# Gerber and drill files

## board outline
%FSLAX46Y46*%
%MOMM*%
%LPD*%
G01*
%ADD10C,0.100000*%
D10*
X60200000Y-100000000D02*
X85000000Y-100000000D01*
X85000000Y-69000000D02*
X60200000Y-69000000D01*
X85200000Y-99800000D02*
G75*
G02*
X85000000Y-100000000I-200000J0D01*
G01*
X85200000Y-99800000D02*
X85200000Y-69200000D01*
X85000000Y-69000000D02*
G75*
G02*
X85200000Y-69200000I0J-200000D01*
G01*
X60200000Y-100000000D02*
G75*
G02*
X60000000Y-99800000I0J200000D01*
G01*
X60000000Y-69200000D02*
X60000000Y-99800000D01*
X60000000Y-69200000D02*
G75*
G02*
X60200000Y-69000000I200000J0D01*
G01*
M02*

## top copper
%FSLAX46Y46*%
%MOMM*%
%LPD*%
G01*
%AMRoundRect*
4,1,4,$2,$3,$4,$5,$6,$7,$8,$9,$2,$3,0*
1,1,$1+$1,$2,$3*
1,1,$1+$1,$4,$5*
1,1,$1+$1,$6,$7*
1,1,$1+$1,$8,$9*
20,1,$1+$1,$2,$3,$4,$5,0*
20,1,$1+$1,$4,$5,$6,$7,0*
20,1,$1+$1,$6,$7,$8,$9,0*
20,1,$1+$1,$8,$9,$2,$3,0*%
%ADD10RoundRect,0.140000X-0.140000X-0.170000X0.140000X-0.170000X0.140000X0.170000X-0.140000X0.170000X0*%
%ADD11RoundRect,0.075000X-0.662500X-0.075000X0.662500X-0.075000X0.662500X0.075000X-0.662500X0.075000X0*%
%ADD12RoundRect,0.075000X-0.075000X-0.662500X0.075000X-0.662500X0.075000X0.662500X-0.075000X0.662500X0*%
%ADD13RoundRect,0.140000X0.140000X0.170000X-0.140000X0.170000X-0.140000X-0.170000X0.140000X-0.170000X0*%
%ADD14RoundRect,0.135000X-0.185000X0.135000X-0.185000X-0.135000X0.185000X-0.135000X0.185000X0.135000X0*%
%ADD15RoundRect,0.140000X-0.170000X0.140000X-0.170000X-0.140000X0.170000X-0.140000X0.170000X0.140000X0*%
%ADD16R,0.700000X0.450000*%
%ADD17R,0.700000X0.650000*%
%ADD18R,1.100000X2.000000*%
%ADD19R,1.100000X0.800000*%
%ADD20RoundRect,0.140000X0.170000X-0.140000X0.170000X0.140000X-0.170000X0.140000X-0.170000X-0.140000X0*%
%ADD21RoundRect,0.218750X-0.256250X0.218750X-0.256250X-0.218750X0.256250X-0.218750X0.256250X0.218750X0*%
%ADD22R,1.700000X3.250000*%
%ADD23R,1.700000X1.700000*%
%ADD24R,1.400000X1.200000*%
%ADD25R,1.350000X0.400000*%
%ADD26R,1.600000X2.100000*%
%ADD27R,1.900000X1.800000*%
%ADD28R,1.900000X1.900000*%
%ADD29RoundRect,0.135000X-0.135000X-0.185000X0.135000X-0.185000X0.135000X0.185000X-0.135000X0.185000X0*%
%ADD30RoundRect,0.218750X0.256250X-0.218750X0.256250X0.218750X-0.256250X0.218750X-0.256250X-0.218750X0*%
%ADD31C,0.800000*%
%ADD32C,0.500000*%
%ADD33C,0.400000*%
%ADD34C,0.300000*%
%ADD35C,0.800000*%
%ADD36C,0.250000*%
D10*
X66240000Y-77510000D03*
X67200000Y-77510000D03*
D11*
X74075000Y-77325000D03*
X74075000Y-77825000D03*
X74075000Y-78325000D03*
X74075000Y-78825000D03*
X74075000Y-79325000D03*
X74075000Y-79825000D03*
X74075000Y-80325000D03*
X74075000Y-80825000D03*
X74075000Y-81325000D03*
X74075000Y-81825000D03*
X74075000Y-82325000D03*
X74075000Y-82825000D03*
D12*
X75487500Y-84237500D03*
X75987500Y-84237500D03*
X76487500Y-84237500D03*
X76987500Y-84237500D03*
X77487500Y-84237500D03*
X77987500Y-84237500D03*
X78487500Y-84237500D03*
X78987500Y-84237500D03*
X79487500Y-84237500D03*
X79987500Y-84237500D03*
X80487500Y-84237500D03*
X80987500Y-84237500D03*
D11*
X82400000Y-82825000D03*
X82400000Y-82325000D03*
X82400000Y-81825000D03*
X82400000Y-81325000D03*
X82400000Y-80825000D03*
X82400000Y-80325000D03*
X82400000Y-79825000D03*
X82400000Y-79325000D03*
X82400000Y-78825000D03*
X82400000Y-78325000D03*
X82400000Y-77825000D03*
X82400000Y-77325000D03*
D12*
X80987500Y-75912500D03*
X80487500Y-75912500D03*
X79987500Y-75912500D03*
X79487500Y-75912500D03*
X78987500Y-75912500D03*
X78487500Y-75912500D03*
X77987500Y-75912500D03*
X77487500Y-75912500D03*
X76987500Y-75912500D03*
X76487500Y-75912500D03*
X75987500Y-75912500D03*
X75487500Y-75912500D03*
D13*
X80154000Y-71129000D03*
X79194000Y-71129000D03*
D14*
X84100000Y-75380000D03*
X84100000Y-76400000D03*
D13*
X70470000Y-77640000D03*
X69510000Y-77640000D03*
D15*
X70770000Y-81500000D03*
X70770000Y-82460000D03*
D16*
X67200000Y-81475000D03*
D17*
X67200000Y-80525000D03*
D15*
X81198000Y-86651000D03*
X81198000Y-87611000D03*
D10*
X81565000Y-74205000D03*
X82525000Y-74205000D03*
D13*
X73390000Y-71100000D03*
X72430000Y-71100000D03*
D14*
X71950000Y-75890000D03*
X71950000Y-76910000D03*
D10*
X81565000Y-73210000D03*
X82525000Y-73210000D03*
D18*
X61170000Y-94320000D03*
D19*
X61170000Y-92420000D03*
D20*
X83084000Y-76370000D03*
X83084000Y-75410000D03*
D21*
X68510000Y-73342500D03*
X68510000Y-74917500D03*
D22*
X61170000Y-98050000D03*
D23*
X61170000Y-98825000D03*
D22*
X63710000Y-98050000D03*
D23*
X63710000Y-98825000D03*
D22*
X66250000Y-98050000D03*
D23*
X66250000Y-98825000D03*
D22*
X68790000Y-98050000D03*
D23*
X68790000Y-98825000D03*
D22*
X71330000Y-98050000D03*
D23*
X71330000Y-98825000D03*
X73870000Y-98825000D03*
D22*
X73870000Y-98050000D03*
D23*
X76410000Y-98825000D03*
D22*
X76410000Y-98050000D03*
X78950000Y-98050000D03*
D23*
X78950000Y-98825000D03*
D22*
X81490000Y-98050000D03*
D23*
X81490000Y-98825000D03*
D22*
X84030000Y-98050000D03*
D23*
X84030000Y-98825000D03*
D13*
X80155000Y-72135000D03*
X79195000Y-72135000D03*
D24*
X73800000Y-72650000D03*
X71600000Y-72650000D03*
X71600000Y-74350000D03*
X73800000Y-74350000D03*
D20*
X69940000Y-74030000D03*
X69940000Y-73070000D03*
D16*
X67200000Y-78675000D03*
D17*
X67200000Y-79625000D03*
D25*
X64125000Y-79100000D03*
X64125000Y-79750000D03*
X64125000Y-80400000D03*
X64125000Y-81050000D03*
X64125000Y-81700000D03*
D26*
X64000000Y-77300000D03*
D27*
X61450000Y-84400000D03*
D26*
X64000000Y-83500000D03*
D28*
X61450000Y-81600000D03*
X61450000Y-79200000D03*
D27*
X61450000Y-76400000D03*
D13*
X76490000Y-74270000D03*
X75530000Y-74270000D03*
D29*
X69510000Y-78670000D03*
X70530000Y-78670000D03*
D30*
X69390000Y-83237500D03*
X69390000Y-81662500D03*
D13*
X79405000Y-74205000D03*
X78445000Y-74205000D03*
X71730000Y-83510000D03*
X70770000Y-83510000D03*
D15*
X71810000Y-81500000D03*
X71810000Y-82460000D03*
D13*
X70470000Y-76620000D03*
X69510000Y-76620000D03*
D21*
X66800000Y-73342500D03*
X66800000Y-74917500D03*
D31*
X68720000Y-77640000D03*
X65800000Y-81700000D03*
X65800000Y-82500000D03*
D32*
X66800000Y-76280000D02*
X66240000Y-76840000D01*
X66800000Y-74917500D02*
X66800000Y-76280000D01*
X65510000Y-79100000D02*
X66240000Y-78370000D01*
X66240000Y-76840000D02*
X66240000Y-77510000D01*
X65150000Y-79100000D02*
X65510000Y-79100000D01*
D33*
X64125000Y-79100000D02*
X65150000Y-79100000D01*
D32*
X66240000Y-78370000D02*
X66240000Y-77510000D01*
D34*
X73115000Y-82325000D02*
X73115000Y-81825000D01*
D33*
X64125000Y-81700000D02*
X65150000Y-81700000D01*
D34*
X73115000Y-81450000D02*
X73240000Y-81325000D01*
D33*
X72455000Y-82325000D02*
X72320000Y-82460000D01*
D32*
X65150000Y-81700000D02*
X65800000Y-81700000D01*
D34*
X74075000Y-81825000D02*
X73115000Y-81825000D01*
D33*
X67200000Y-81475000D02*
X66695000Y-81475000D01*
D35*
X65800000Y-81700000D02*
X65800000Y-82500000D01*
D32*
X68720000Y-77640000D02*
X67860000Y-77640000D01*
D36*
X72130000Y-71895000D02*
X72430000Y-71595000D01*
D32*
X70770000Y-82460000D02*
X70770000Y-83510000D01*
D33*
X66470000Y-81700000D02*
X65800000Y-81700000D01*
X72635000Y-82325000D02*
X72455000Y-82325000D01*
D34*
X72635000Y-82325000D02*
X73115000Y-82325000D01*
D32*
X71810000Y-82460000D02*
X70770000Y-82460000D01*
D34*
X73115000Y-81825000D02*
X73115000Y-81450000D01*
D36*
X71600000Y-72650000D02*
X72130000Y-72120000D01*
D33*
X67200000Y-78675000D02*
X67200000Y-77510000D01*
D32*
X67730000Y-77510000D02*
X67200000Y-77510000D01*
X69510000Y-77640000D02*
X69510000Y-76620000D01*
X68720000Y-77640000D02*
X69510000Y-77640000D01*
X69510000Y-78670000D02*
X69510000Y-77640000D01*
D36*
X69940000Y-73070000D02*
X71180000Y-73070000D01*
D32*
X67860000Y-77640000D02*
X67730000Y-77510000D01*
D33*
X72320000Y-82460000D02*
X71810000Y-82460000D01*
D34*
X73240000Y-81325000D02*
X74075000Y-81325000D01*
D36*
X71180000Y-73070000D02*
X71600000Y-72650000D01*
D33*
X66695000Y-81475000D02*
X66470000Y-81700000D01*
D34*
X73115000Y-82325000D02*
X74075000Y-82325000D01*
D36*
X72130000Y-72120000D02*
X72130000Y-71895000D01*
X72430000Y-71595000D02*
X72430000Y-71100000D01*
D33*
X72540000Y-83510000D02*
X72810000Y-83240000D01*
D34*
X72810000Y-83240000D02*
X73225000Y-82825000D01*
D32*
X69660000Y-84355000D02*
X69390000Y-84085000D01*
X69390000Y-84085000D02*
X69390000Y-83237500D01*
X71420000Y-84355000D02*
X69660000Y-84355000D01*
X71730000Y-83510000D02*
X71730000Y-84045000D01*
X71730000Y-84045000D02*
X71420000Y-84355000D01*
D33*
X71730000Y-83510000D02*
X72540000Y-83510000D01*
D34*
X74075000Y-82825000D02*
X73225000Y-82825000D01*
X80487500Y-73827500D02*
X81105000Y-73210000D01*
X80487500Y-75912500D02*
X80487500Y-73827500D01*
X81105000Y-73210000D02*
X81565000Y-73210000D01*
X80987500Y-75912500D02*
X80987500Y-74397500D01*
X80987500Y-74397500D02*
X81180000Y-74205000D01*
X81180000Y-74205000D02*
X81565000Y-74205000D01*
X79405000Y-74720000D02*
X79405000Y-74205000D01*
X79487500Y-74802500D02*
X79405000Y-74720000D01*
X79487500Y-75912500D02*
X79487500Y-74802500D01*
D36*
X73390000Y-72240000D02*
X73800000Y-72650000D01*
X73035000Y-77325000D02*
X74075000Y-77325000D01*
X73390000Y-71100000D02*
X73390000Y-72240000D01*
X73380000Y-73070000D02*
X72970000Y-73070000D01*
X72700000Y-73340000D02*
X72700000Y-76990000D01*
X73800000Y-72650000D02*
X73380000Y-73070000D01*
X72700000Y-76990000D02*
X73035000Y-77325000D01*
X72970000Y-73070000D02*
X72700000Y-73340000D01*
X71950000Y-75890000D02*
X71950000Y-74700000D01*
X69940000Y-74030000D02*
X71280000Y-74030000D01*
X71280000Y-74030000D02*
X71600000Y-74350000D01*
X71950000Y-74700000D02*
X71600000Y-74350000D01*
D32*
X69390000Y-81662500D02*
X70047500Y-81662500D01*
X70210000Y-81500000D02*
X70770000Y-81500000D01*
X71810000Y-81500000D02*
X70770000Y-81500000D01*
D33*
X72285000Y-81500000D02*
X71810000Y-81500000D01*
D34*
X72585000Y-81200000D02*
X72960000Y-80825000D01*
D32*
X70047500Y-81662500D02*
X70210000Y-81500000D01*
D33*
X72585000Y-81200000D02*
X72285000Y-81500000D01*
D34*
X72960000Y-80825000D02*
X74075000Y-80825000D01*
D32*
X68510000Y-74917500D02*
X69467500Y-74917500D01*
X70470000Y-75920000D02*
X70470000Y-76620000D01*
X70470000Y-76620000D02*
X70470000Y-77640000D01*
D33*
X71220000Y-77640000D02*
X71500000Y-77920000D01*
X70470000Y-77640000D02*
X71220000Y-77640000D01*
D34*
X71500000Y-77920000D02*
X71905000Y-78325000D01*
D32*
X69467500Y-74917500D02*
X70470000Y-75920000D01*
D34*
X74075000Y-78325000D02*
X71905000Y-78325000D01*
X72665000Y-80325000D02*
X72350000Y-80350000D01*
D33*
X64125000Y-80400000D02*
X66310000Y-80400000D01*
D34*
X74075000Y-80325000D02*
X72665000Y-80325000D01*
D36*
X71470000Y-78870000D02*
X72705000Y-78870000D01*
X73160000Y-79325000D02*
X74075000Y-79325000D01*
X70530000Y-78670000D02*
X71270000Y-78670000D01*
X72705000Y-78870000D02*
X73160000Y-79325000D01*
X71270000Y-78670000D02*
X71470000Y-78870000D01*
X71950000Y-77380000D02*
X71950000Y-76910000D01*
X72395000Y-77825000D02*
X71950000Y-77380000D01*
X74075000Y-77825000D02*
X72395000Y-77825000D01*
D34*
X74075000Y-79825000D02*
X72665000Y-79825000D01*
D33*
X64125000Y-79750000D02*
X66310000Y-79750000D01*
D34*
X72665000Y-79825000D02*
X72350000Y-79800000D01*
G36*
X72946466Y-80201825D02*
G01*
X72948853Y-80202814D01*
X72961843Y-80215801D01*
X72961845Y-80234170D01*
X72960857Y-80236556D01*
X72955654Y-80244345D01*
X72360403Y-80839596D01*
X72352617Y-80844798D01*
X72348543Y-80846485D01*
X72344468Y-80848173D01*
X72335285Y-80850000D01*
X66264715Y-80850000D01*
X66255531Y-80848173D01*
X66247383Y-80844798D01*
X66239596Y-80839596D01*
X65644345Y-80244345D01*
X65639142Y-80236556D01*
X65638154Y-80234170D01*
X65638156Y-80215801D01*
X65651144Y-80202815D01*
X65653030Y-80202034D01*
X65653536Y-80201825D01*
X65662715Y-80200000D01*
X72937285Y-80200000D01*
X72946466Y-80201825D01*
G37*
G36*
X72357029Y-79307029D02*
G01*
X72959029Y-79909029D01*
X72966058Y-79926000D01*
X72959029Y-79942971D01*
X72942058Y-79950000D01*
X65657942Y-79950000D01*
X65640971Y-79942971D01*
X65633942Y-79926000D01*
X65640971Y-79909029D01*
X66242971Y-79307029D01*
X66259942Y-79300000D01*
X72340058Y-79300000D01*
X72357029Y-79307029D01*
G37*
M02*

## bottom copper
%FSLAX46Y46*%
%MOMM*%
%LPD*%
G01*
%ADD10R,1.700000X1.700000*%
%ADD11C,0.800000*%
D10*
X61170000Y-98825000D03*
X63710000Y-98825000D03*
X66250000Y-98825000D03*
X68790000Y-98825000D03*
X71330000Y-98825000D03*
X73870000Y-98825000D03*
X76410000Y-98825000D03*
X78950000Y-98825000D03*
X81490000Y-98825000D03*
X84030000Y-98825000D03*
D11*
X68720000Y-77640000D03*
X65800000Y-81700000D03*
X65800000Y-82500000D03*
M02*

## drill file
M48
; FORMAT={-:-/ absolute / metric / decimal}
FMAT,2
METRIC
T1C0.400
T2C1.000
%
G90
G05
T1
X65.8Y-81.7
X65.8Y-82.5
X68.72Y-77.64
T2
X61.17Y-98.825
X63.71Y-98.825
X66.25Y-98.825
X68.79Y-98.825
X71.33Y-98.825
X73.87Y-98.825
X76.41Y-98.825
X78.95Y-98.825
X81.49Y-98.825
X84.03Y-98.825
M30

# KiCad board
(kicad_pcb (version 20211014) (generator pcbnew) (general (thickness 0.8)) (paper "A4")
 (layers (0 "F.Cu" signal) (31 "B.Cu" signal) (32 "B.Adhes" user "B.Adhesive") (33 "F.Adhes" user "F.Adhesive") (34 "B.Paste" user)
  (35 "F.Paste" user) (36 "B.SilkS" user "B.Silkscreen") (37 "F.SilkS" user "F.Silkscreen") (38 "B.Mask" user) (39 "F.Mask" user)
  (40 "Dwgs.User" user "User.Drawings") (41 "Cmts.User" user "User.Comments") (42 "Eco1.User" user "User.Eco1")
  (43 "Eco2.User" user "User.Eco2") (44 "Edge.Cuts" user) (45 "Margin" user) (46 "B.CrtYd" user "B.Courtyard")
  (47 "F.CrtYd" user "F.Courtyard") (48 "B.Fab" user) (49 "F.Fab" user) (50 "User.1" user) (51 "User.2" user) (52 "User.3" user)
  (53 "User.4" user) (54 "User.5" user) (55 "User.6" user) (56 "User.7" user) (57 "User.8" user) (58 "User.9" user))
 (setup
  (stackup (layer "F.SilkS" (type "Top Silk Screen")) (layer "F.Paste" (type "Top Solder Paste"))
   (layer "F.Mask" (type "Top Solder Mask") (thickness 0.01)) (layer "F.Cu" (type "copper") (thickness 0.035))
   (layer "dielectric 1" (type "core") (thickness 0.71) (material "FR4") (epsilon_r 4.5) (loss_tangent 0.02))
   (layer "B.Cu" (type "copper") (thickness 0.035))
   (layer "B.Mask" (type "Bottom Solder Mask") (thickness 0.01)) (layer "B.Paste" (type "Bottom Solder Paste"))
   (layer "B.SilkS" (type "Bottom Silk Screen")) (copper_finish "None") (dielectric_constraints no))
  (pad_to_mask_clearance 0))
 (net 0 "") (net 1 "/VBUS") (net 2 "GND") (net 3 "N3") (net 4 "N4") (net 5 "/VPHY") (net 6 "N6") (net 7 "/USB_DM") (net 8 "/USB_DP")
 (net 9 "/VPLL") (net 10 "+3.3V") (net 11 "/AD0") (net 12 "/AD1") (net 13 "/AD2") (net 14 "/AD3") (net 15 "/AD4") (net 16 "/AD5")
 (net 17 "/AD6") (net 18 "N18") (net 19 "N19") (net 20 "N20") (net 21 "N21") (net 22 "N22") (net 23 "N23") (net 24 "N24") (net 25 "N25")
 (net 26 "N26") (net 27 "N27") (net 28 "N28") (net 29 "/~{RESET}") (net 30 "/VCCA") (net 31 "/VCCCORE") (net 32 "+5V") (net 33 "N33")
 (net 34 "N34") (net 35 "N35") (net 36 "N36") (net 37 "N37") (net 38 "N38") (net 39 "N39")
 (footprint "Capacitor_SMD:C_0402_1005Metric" (layer "F.Cu") (at 66.72 77.51)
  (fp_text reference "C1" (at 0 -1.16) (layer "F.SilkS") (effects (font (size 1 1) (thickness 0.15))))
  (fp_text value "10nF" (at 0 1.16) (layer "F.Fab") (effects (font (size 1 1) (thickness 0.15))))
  (pad "1" smd roundrect (at -0.48 0) (size 0.56 0.62) (layers "F.Cu" "F.Paste" "F.Mask") (roundrect_rratio 0.25) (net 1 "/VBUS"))
  (pad "2" smd roundrect (at 0.48 0) (size 0.56 0.62) (layers "F.Cu" "F.Paste" "F.Mask") (roundrect_rratio 0.25) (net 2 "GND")))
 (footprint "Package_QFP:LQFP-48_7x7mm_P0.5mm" (layer "F.Cu") (at 78.2375 80.075)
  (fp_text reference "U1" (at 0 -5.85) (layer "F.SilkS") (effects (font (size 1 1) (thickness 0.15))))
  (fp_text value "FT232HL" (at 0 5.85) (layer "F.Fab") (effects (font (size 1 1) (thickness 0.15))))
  (pad "1" smd roundrect (at -4.1625 -2.75) (size 1.475 0.3) (layers "F.Cu" "F.Paste" "F.Mask") (roundrect_rratio 0.25) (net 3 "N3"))
  (pad "2" smd roundrect (at -4.1625 -2.25) (size 1.475 0.3) (layers "F.Cu" "F.Paste" "F.Mask") (roundrect_rratio 0.25) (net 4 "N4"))
  (pad "3" smd roundrect (at -4.1625 -1.75) (size 1.475 0.3) (layers "F.Cu" "F.Paste" "F.Mask") (roundrect_rratio 0.25) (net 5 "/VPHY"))
  (pad "4" smd roundrect (at -4.1625 -1.25) (size 1.475 0.3) (layers "F.Cu" "F.Paste" "F.Mask") (roundrect_rratio 0.25) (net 2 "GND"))
  (pad "5" smd roundrect (at -4.1625 -0.75) (size 1.475 0.3) (layers "F.Cu" "F.Paste" "F.Mask") (roundrect_rratio 0.25) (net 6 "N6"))
  (pad "6" smd roundrect (at -4.1625 -0.25) (size 1.475 0.3) (layers "F.Cu" "F.Paste" "F.Mask") (roundrect_rratio 0.25) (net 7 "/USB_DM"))
  (pad "7" smd roundrect (at -4.1625 0.25) (size 1.475 0.3) (layers "F.Cu" "F.Paste" "F.Mask") (roundrect_rratio 0.25) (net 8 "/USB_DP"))
  (pad "8" smd roundrect (at -4.1625 0.75) (size 1.475 0.3) (layers "F.Cu" "F.Paste" "F.Mask") (roundrect_rratio 0.25) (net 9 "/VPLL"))
  (pad "9" smd roundrect (at -4.1625 1.25) (size 1.475 0.3) (layers "F.Cu" "F.Paste" "F.Mask") (roundrect_rratio 0.25) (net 2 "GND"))
  (pad "10" smd roundrect (at -4.1625 1.75) (size 1.475 0.3) (layers "F.Cu" "F.Paste" "F.Mask") (roundrect_rratio 0.25) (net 2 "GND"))
  (pad "11" smd roundrect (at -4.1625 2.25) (size 1.475 0.3) (layers "F.Cu" "F.Paste" "F.Mask") (roundrect_rratio 0.25) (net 2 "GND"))
  (pad "12" smd roundrect (at -4.1625 2.75) (size 1.475 0.3) (layers "F.Cu" "F.Paste" "F.Mask") (roundrect_rratio 0.25) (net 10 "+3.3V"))
  (pad "13" smd roundrect (at -2.75 4.1625) (size 0.3 1.475) (layers "F.Cu" "F.Paste" "F.Mask") (roundrect_rratio 0.25) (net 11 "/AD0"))
  (pad "14" smd roundrect (at -2.25 4.1625) (size 0.3 1.475) (layers "F.Cu" "F.Paste" "F.Mask") (roundrect_rratio 0.25) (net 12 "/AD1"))
  (pad "15" smd roundrect (at -1.75 4.1625) (size 0.3 1.475) (layers "F.Cu" "F.Paste" "F.Mask") (roundrect_rratio 0.25) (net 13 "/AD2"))
  (pad "16" smd roundrect (at -1.25 4.1625) (size 0.3 1.475) (layers "F.Cu" "F.Paste" "F.Mask") (roundrect_rratio 0.25) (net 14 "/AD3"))
  (pad "17" smd roundrect (at -0.75 4.1625) (size 0.3 1.475) (layers "F.Cu" "F.Paste" "F.Mask") (roundrect_rratio 0.25) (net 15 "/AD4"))
  (pad "18" smd roundrect (at -0.25 4.1625) (size 0.3 1.475) (layers "F.Cu" "F.Paste" "F.Mask") (roundrect_rratio 0.25) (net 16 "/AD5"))
  (pad "19" smd roundrect (at 0.25 4.1625) (size 0.3 1.475) (layers "F.Cu" "F.Paste" "F.Mask") (roundrect_rratio 0.25) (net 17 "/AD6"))
  (pad "20" smd roundrect (at 0.75 4.1625) (size 0.3 1.475) (layers "F.Cu" "F.Paste" "F.Mask") (roundrect_rratio 0.25) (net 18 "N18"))
  (pad "21" smd roundrect (at 1.25 4.1625) (size 0.3 1.475) (layers "F.Cu" "F.Paste" "F.Mask") (roundrect_rratio 0.25) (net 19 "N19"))
  (pad "22" smd roundrect (at 1.75 4.1625) (size 0.3 1.475) (layers "F.Cu" "F.Paste" "F.Mask") (roundrect_rratio 0.25) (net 2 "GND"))
  (pad "23" smd roundrect (at 2.25 4.1625) (size 0.3 1.475) (layers "F.Cu" "F.Paste" "F.Mask") (roundrect_rratio 0.25) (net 2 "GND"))
  (pad "24" smd roundrect (at 2.75 4.1625) (size 0.3 1.475) (layers "F.Cu" "F.Paste" "F.Mask") (roundrect_rratio 0.25) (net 10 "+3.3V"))
  (pad "25" smd roundrect (at 4.1625 2.75) (size 1.475 0.3) (layers "F.Cu" "F.Paste" "F.Mask") (roundrect_rratio 0.25) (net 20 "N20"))
  (pad "26" smd roundrect (at 4.1625 2.25) (size 1.475 0.3) (layers "F.Cu" "F.Paste" "F.Mask") (roundrect_rratio 0.25) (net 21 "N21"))
  (pad "27" smd roundrect (at 4.1625 1.75) (size 1.475 0.3) (layers "F.Cu" "F.Paste" "F.Mask") (roundrect_rratio 0.25) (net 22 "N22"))
  (pad "28" smd roundrect (at 4.1625 1.25) (size 1.475 0.3) (layers "F.Cu" "F.Paste" "F.Mask") (roundrect_rratio 0.25) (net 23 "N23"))
  (pad "29" smd roundrect (at 4.1625 0.75) (size 1.475 0.3) (layers "F.Cu" "F.Paste" "F.Mask") (roundrect_rratio 0.25) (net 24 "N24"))
  (pad "30" smd roundrect (at 4.1625 0.25) (size 1.475 0.3) (layers "F.Cu" "F.Paste" "F.Mask") (roundrect_rratio 0.25) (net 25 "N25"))
  (pad "31" smd roundrect (at 4.1625 -0.25) (size 1.475 0.3) (layers "F.Cu" "F.Paste" "F.Mask") (roundrect_rratio 0.25) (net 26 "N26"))
  (pad "32" smd roundrect (at 4.1625 -0.75) (size 1.475 0.3) (layers "F.Cu" "F.Paste" "F.Mask") (roundrect_rratio 0.25) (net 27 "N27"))
  (pad "33" smd roundrect (at 4.1625 -1.25) (size 1.475 0.3) (layers "F.Cu" "F.Paste" "F.Mask") (roundrect_rratio 0.25) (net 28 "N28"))
  (pad "34" smd roundrect (at 4.1625 -1.75) (size 1.475 0.3) (layers "F.Cu" "F.Paste" "F.Mask") (roundrect_rratio 0.25) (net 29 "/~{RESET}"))
  (pad "35" smd roundrect (at 4.1625 -2.25) (size 1.475 0.3) (layers "F.Cu" "F.Paste" "F.Mask") (roundrect_rratio 0.25) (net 2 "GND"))
  (pad "36" smd roundrect (at 4.1625 -2.75) (size 1.475 0.3) (layers "F.Cu" "F.Paste" "F.Mask") (roundrect_rratio 0.25) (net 2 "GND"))
  (pad "37" smd roundrect (at 2.75 -4.1625) (size 0.3 1.475) (layers "F.Cu" "F.Paste" "F.Mask") (roundrect_rratio 0.25) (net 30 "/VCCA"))
  (pad "38" smd roundrect (at 2.25 -4.1625) (size 0.3 1.475) (layers "F.Cu" "F.Paste" "F.Mask") (roundrect_rratio 0.25) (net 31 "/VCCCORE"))
  (pad "39" smd roundrect (at 1.75 -4.1625) (size 0.3 1.475) (layers "F.Cu" "F.Paste" "F.Mask") (roundrect_rratio 0.25) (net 10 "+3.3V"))
  (pad "40" smd roundrect (at 1.25 -4.1625) (size 0.3 1.475) (layers "F.Cu" "F.Paste" "F.Mask") (roundrect_rratio 0.25) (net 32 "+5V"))
  (pad "41" smd roundrect (at 0.75 -4.1625) (size 0.3 1.475) (layers "F.Cu" "F.Paste" "F.Mask") (roundrect_rratio 0.25) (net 2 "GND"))
  (pad "42" smd roundrect (at 0.25 -4.1625) (size 0.3 1.475) (layers "F.Cu" "F.Paste" "F.Mask") (roundrect_rratio 0.25) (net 2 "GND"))
  (pad "43" smd roundrect (at -0.25 -4.1625) (size 0.3 1.475) (layers "F.Cu" "F.Paste" "F.Mask") (roundrect_rratio 0.25) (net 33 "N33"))
  (pad "44" smd roundrect (at -0.75 -4.1625) (size 0.3 1.475) (layers "F.Cu" "F.Paste" "F.Mask") (roundrect_rratio 0.25) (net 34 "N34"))
  (pad "45" smd roundrect (at -1.25 -4.1625) (size 0.3 1.475) (layers "F.Cu" "F.Paste" "F.Mask") (roundrect_rratio 0.25) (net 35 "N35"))
  (pad "46" smd roundrect (at -1.75 -4.1625) (size 0.3 1.475) (layers "F.Cu" "F.Paste" "F.Mask") (roundrect_rratio 0.25) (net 10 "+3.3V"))
  (pad "47" smd roundrect (at -2.25 -4.1625) (size 0.3 1.475) (layers "F.Cu" "F.Paste" "F.Mask") (roundrect_rratio 0.25) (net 2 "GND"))
  (pad "48" smd roundrect (at -2.75 -4.1625) (size 0.3 1.475) (layers "F.Cu" "F.Paste" "F.Mask") (roundrect_rratio 0.25) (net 2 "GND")))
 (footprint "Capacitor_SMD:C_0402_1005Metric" (layer "F.Cu") (at 79.674 71.129 180)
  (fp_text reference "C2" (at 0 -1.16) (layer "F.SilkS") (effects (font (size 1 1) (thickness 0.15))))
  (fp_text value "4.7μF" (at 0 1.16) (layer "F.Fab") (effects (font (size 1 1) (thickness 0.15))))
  (pad "1" smd roundrect (at -0.48 0 180) (size 0.56 0.62) (layers "F.Cu" "F.Paste" "F.Mask") (roundrect_rratio 0.25) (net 10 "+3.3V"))
  (pad "2" smd roundrect (at 0.48 0 180) (size 0.56 0.62) (layers "F.Cu" "F.Paste" "F.Mask") (roundrect_rratio 0.25) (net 2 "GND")))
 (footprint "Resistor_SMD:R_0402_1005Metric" (layer "F.Cu") (at 84.1 75.89 -90)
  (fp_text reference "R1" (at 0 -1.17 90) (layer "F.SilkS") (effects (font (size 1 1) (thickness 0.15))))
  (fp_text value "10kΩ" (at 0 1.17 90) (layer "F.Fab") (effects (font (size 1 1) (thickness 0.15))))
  (pad "1" smd roundrect (at -0.51 0 270) (size 0.54 0.64) (layers "F.Cu" "F.Paste" "F.Mask") (roundrect_rratio 0.25) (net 10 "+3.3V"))
  (pad "2" smd roundrect (at 0.51 0 270) (size 0.54 0.64) (layers "F.Cu" "F.Paste" "F.Mask") (roundrect_rratio 0.25) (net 29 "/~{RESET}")))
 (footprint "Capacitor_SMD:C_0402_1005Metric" (layer "F.Cu") (at 69.99 77.64 180)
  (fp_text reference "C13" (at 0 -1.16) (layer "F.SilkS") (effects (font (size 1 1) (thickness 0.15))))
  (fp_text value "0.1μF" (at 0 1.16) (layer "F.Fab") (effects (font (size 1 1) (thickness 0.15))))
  (pad "1" smd roundrect (at -0.48 0 180) (size 0.56 0.62) (layers "F.Cu" "F.Paste" "F.Mask") (roundrect_rratio 0.25) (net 5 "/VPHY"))
  (pad "2" smd roundrect (at 0.48 0 180) (size 0.56 0.62) (layers "F.Cu" "F.Paste" "F.Mask") (roundrect_rratio 0.25) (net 2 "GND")))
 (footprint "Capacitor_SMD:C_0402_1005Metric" (layer "F.Cu") (at 70.77 81.98 -90)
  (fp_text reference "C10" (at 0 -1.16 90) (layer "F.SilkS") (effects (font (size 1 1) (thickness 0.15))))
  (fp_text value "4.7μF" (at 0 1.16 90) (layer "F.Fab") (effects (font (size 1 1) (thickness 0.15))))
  (pad "1" smd roundrect (at -0.48 0 270) (size 0.56 0.62) (layers "F.Cu" "F.Paste" "F.Mask") (roundrect_rratio 0.25) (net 9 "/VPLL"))
  (pad "2" smd roundrect (at 0.48 0 270) (size 0.56 0.62) (layers "F.Cu" "F.Paste" "F.Mask") (roundrect_rratio 0.25) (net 2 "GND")))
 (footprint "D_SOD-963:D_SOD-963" (layer "F.Cu") (at 67.2 80.95 90)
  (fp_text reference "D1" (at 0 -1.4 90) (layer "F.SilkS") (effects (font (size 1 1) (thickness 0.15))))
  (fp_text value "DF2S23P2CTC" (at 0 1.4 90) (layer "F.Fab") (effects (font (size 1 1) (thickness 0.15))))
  (pad "1" smd rect (at -0.525 0 270) (size 0.45 0.7) (layers "F.Cu" "F.Paste" "F.Mask") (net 2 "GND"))
  (pad "2" smd rect (at 0.425 0 270) (size 0.65 0.7) (layers "F.Cu" "F.Paste" "F.Mask") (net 8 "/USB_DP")))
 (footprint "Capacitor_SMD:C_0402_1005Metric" (layer "F.Cu") (at 81.198 87.131 -90)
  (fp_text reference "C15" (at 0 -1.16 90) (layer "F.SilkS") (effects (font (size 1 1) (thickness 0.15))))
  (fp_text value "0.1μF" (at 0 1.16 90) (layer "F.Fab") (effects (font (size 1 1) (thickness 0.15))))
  (pad "1" smd roundrect (at -0.48 0 270) (size 0.56 0.62) (layers "F.Cu" "F.Paste" "F.Mask") (roundrect_rratio 0.25) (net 10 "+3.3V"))
  (pad "2" smd roundrect (at 0.48 0 270) (size 0.56 0.62) (layers "F.Cu" "F.Paste" "F.Mask") (roundrect_rratio 0.25) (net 2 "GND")))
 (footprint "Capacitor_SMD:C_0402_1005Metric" (layer "F.Cu") (at 82.045 74.205)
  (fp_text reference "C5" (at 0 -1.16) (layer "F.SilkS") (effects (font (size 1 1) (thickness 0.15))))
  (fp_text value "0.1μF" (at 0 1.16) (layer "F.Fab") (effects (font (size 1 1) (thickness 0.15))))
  (pad "1" smd roundrect (at -0.48 0) (size 0.56 0.62) (layers "F.Cu" "F.Paste" "F.Mask") (roundrect_rratio 0.25) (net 30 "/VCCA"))
  (pad "2" smd roundrect (at 0.48 0) (size 0.56 0.62) (layers "F.Cu" "F.Paste" "F.Mask") (roundrect_rratio 0.25) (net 2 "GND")))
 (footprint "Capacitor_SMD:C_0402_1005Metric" (layer "F.Cu") (at 72.91 71.1 180)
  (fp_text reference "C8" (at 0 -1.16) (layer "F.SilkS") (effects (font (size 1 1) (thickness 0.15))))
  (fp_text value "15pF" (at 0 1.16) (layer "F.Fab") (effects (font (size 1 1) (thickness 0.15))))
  (pad "1" smd roundrect (at -0.48 0 180) (size 0.56 0.62) (layers "F.Cu" "F.Paste" "F.Mask") (roundrect_rratio 0.25) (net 3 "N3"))
  (pad "2" smd roundrect (at 0.48 0 180) (size 0.56 0.62) (layers "F.Cu" "F.Paste" "F.Mask") (roundrect_rratio 0.25) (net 2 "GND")))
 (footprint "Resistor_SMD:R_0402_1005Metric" (layer "F.Cu") (at 71.95 76.4 -90)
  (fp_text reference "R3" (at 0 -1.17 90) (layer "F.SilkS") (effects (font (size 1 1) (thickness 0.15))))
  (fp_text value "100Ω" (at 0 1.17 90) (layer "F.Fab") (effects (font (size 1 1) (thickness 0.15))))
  (pad "1" smd roundrect (at -0.51 0 270) (size 0.54 0.64) (layers "F.Cu" "F.Paste" "F.Mask") (roundrect_rratio 0.25) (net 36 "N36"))
  (pad "2" smd roundrect (at 0.51 0 270) (size 0.54 0.64) (layers "F.Cu" "F.Paste" "F.Mask") (roundrect_rratio 0.25) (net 4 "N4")))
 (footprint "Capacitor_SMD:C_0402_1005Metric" (layer "F.Cu") (at 82.045 73.21)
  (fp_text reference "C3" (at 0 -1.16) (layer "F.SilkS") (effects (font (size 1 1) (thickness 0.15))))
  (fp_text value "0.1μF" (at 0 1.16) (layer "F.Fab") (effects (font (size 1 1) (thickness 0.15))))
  (pad "1" smd roundrect (at -0.48 0) (size 0.56 0.62) (layers "F.Cu" "F.Paste" "F.Mask") (roundrect_rratio 0.25) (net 31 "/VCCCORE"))
  (pad "2" smd roundrect (at 0.48 0) (size 0.56 0.62) (layers "F.Cu" "F.Paste" "F.Mask") (roundrect_rratio 0.25) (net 2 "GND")))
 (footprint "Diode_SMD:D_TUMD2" (layer "F.Cu") (at 61.17 93.67 90)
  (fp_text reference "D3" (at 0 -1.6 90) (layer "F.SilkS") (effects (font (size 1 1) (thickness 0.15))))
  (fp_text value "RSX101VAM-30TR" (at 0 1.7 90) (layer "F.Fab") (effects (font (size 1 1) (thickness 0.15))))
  (pad "1" smd rect (at -0.65 0 270) (size 2 1.1) (layers "F.Cu" "F.Paste" "F.Mask") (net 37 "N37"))
  (pad "2" smd rect (at 1.25 0 270) (size 0.8 1.1) (layers "F.Cu" "F.Paste" "F.Mask") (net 32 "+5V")))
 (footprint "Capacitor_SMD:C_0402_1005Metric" (layer "F.Cu") (at 83.084 75.89 90)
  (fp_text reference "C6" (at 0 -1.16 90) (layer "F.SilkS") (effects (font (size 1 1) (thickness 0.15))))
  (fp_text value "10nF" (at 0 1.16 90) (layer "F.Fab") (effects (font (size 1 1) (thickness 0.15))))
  (pad "1" smd roundrect (at -0.48 0 90) (size 0.56 0.62) (layers "F.Cu" "F.Paste" "F.Mask") (roundrect_rratio 0.25) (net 29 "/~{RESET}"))
  (pad "2" smd roundrect (at 0.48 0 90) (size 0.56 0.62) (layers "F.Cu" "F.Paste" "F.Mask") (roundrect_rratio 0.25) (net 2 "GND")))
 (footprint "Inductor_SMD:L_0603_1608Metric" (layer "F.Cu") (at 68.51 74.13 -90)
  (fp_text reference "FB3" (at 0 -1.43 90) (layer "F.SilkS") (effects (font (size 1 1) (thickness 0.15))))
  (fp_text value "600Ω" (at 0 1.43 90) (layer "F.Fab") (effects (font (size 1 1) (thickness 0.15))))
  (pad "1" smd roundrect (at -0.7875 0 270) (size 0.875 0.95) (layers "F.Cu" "F.Paste" "F.Mask") (roundrect_rratio 0.25) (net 10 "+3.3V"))
  (pad "2" smd roundrect (at 0.7875 0 270) (size 0.875 0.95) (layers "F.Cu" "F.Paste" "F.Mask") (roundrect_rratio 0.25) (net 5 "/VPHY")))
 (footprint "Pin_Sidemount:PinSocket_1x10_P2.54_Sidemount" (layer "F.Cu") (at 61.17 98.05)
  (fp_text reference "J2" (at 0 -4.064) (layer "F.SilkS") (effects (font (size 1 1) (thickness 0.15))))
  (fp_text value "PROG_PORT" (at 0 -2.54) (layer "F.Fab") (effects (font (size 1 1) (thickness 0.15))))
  (pad "1" smd rect (at 0 0) (size 1.7 3.25) (layers "F.Cu" "F.Mask") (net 37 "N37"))
  (pad "1" thru_hole rect (at 0 0.775) (size 1.7 1.7) (drill 1) (layers *.Cu *.Mask) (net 37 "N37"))
  (pad "2" smd rect (at 2.54 0) (size 1.7 3.25) (layers "F.Cu" "F.Mask") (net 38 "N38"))
  (pad "2" thru_hole rect (at 2.54 0.775) (size 1.7 1.7) (drill 1) (layers *.Cu *.Mask) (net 38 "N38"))
  (pad "3" smd rect (at 5.08 0) (size 1.7 3.25) (layers "F.Cu" "F.Mask") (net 2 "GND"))
  (pad "3" thru_hole rect (at 5.08 0.775) (size 1.7 1.7) (drill 1) (layers *.Cu *.Mask) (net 2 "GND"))
  (pad "4" smd rect (at 7.62 0) (size 1.7 3.25) (layers "F.Cu" "F.Mask") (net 11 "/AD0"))
  (pad "4" thru_hole rect (at 7.62 0.775) (size 1.7 1.7) (drill 1) (layers *.Cu *.Mask) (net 11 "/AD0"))
  (pad "5" smd rect (at 10.16 0) (size 1.7 3.25) (layers "F.Cu" "F.Mask") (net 12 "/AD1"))
  (pad "5" thru_hole rect (at 10.16 0.775) (size 1.7 1.7) (drill 1) (layers *.Cu *.Mask) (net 12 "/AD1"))
  (pad "6" thru_hole rect (at 12.7 0.775) (size 1.7 1.7) (drill 1) (layers *.Cu *.Mask) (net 13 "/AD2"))
  (pad "6" smd rect (at 12.7 0) (size 1.7 3.25) (layers "F.Cu" "F.Mask") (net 13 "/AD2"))
  (pad "7" thru_hole rect (at 15.24 0.775) (size 1.7 1.7) (drill 1) (layers *.Cu *.Mask) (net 14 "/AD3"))
  (pad "7" smd rect (at 15.24 0) (size 1.7 3.25) (layers "F.Cu" "F.Mask") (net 14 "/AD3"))
  (pad "8" smd rect (at 17.78 0) (size 1.7 3.25) (layers "F.Cu" "F.Mask") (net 15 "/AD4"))
  (pad "8" thru_hole rect (at 17.78 0.775) (size 1.7 1.7) (drill 1) (layers *.Cu *.Mask) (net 15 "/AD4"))
  (pad "9" smd rect (at 20.32 0) (size 1.7 3.25) (layers "F.Cu" "F.Mask") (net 16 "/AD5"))
  (pad "9" thru_hole rect (at 20.32 0.775) (size 1.7 1.7) (drill 1) (layers *.Cu *.Mask) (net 16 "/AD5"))
  (pad "10" smd rect (at 22.86 0) (size 1.7 3.25) (layers "F.Cu" "F.Mask") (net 17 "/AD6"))
  (pad "10" thru_hole rect (at 22.86 0.775) (size 1.7 1.7) (drill 1) (layers *.Cu *.Mask) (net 17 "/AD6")))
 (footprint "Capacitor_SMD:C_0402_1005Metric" (layer "F.Cu") (at 79.675 72.135 180)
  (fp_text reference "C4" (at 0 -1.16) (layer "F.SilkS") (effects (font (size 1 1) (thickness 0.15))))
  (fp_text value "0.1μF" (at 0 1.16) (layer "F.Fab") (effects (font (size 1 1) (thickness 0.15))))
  (pad "1" smd roundrect (at -0.48 0 180) (size 0.56 0.62) (layers "F.Cu" "F.Paste" "F.Mask") (roundrect_rratio 0.25) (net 10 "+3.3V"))
  (pad "2" smd roundrect (at 0.48 0 180) (size 0.56 0.62) (layers "F.Cu" "F.Paste" "F.Mask") (roundrect_rratio 0.25) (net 2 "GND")))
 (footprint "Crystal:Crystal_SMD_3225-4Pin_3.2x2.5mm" (layer "F.Cu") (at 72.7 73.5 180)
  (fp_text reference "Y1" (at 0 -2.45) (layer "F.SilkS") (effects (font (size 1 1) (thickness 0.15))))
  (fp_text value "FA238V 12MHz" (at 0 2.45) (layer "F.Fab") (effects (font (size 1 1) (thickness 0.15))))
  (pad "1" smd rect (at -1.1 0.85 180) (size 1.4 1.2) (layers "F.Cu" "F.Paste" "F.Mask") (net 3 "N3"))
  (pad "2" smd rect (at 1.1 0.85 180) (size 1.4 1.2) (layers "F.Cu" "F.Paste" "F.Mask") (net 2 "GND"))
  (pad "3" smd rect (at 1.1 -0.85 180) (size 1.4 1.2) (layers "F.Cu" "F.Paste" "F.Mask") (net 36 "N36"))
  (pad "4" smd rect (at -1.1 -0.85 180) (size 1.4 1.2) (layers "F.Cu" "F.Paste" "F.Mask") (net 2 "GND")))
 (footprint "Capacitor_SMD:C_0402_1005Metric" (layer "F.Cu") (at 69.94 73.55 90)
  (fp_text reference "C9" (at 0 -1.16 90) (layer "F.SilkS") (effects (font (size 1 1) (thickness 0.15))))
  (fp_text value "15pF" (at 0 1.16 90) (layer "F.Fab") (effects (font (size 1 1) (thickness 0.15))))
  (pad "1" smd roundrect (at -0.48 0 90) (size 0.56 0.62) (layers "F.Cu" "F.Paste" "F.Mask") (roundrect_rratio 0.25) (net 36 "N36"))
  (pad "2" smd roundrect (at 0.48 0 90) (size 0.56 0.62) (layers "F.Cu" "F.Paste" "F.Mask") (roundrect_rratio 0.25) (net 2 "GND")))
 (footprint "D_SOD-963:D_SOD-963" (layer "F.Cu") (at 67.2 79.2 -90)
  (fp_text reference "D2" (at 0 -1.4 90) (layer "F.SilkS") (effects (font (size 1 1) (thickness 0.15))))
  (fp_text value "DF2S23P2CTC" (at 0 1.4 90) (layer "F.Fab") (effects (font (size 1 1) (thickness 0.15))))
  (pad "1" smd rect (at -0.525 0 90) (size 0.45 0.7) (layers "F.Cu" "F.Paste" "F.Mask") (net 2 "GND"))
  (pad "2" smd rect (at 0.425 0 90) (size 0.65 0.7) (layers "F.Cu" "F.Paste" "F.Mask") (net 7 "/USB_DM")))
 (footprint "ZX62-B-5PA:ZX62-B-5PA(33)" (layer "F.Cu") (at 60 80.4 -90)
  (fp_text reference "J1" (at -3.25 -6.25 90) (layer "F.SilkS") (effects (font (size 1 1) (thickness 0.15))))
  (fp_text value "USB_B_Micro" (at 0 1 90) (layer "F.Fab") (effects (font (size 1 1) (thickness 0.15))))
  (pad "1" smd rect locked (at -1.3 -4.125 270) (size 0.4 1.35) (layers "F.Cu" "F.Paste" "F.Mask") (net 1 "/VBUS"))
  (pad "2" smd rect locked (at -0.65 -4.125 270) (size 0.4 1.35) (layers "F.Cu" "F.Paste" "F.Mask") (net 7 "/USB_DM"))
  (pad "3" smd rect locked (at 0 -4.125 270) (size 0.4 1.35) (layers "F.Cu" "F.Paste" "F.Mask") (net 8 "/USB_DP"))
  (pad "4" smd rect locked (at 0.65 -4.125 270) (size 0.4 1.35) (layers "F.Cu" "F.Paste" "F.Mask") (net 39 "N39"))
  (pad "5" smd rect locked (at 1.3 -4.125 270) (size 0.4 1.35) (layers "F.Cu" "F.Paste" "F.Mask") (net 2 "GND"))
  (pad "6" smd rect locked (at -3.1 -4 270) (size 2.1 1.6) (layers "F.Cu" "F.Paste" "F.Mask") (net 2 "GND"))
  (pad "6" smd rect locked (at 4 -1.45 270) (size 1.8 1.9) (layers "F.Cu" "F.Paste" "F.Mask") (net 2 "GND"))
  (pad "6" smd rect locked (at 3.1 -4 270) (size 2.1 1.6) (layers "F.Cu" "F.Paste" "F.Mask") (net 2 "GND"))
  (pad "6" smd rect locked (at 1.2 -1.45 270) (size 1.9 1.9) (layers "F.Cu" "F.Paste" "F.Mask") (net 2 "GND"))
  (pad "6" smd rect locked (at -1.2 -1.45 270) (size 1.9 1.9) (layers "F.Cu" "F.Paste" "F.Mask") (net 2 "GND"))
  (pad "6" smd rect locked (at -4 -1.45 270) (size 1.8 1.9) (layers "F.Cu" "F.Paste" "F.Mask") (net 2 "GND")))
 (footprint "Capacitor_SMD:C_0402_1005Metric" (layer "F.Cu") (at 76.01 74.27 180)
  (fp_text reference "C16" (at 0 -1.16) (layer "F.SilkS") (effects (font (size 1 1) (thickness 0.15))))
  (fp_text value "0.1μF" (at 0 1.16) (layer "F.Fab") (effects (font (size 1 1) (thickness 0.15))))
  (pad "1" smd roundrect (at -0.48 0 180) (size 0.56 0.62) (layers "F.Cu" "F.Paste" "F.Mask") (roundrect_rratio 0.25) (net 10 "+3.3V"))
  (pad "2" smd roundrect (at 0.48 0 180) (size 0.56 0.62) (layers "F.Cu" "F.Paste" "F.Mask") (roundrect_rratio 0.25) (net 2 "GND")))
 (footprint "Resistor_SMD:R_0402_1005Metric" (layer "F.Cu") (at 70.02 78.67)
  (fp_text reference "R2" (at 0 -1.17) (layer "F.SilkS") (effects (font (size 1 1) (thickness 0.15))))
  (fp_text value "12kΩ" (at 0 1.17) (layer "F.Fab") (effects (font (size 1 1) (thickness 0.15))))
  (pad "1" smd roundrect (at -0.51 0) (size 0.54 0.64) (layers "F.Cu" "F.Paste" "F.Mask") (roundrect_rratio 0.25) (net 2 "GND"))
  (pad "2" smd roundrect (at 0.51 0) (size 0.54 0.64) (layers "F.Cu" "F.Paste" "F.Mask") (roundrect_rratio 0.25) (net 6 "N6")))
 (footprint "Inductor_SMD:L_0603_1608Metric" (layer "F.Cu") (at 69.39 82.45 90)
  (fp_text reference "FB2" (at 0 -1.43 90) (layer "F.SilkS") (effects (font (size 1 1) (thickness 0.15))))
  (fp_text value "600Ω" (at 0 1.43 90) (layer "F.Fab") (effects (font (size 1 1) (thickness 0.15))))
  (pad "1" smd roundrect (at -0.7875 0 90) (size 0.875 0.95) (layers "F.Cu" "F.Paste" "F.Mask") (roundrect_rratio 0.25) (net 10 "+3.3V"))
  (pad "2" smd roundrect (at 0.7875 0 90) (size 0.875 0.95) (layers "F.Cu" "F.Paste" "F.Mask") (roundrect_rratio 0.25) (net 9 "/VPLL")))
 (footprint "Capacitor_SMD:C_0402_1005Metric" (layer "F.Cu") (at 78.925 74.205 180)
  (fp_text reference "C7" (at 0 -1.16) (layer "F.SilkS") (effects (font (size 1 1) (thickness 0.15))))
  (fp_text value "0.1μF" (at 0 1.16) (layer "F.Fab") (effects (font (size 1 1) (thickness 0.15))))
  (pad "1" smd roundrect (at -0.48 0 180) (size 0.56 0.62) (layers "F.Cu" "F.Paste" "F.Mask") (roundrect_rratio 0.25) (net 32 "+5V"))
  (pad "2" smd roundrect (at 0.48 0 180) (size 0.56 0.62) (layers "F.Cu" "F.Paste" "F.Mask") (roundrect_rratio 0.25) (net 2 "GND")))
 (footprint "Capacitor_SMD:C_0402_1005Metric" (layer "F.Cu") (at 71.25 83.51 180)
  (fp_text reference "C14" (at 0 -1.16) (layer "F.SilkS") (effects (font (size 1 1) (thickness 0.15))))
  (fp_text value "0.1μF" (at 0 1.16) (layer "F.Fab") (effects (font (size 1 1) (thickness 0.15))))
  (pad "1" smd roundrect (at -0.48 0 180) (size 0.56 0.62) (layers "F.Cu" "F.Paste" "F.Mask") (roundrect_rratio 0.25) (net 10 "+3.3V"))
  (pad "2" smd roundrect (at 0.48 0 180) (size 0.56 0.62) (layers "F.Cu" "F.Paste" "F.Mask") (roundrect_rratio 0.25) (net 2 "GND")))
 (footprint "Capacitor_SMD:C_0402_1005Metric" (layer "F.Cu") (at 71.81 81.98 -90)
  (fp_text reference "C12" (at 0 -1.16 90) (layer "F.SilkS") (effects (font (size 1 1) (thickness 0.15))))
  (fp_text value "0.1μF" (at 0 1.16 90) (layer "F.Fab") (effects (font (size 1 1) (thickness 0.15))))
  (pad "1" smd roundrect (at -0.48 0 270) (size 0.56 0.62) (layers "F.Cu" "F.Paste" "F.Mask") (roundrect_rratio 0.25) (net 9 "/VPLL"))
  (pad "2" smd roundrect (at 0.48 0 270) (size 0.56 0.62) (layers "F.Cu" "F.Paste" "F.Mask") (roundrect_rratio 0.25) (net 2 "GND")))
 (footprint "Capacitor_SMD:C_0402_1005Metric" (layer "F.Cu") (at 69.99 76.62 180)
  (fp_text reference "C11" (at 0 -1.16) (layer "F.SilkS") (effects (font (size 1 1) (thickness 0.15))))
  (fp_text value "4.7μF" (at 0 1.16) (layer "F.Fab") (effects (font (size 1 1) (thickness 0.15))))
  (pad "1" smd roundrect (at -0.48 0 180) (size 0.56 0.62) (layers "F.Cu" "F.Paste" "F.Mask") (roundrect_rratio 0.25) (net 5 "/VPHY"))
  (pad "2" smd roundrect (at 0.48 0 180) (size 0.56 0.62) (layers "F.Cu" "F.Paste" "F.Mask") (roundrect_rratio 0.25) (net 2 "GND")))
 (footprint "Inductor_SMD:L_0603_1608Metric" (layer "F.Cu") (at 66.8 74.13 -90)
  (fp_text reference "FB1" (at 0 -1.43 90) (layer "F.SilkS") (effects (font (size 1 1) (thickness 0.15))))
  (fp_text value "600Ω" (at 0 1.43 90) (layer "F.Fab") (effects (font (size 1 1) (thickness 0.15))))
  (pad "1" smd roundrect (at -0.7875 0 270) (size 0.875 0.95) (layers "F.Cu" "F.Paste" "F.Mask") (roundrect_rratio 0.25) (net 32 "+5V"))
  (pad "2" smd roundrect (at 0.7875 0 270) (size 0.875 0.95) (layers "F.Cu" "F.Paste" "F.Mask") (roundrect_rratio 0.25) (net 1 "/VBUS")))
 (gr_line (start 60.2 100) (end 85 100) (layer "Edge.Cuts") (width 0.1))
 (gr_line (start 85 69) (end 60.2 69) (layer "Edge.Cuts") (width 0.1))
 (gr_arc (start 85.2 99.8) (mid 85.141421 99.941421) (end 85 100) (layer "Edge.Cuts") (width 0.1))
 (gr_line (start 85.2 99.8) (end 85.2 69.2) (layer "Edge.Cuts") (width 0.1))
 (gr_arc (start 85 69) (mid 85.141421 69.058579) (end 85.2 69.2) (layer "Edge.Cuts") (width 0.1))
 (gr_arc (start 60.2 100) (mid 60.058579 99.941421) (end 60 99.8) (layer "Edge.Cuts") (width 0.1))
 (gr_line (start 60 69.2) (end 60 99.8) (layer "Edge.Cuts") (width 0.1))
 (gr_arc (start 60 69.2) (mid 60.058579 69.058579) (end 60.2 69) (layer "Edge.Cuts") (width 0.1))
 (segment (start 66.8 76.28) (end 66.24 76.84) (width 0.5) (layer "F.Cu") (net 1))
 (segment (start 66.8 74.9175) (end 66.8 76.28) (width 0.5) (layer "F.Cu") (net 1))
 (segment (start 65.51 79.1) (end 66.24 78.37) (width 0.5) (layer "F.Cu") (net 1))
 (segment (start 66.24 76.84) (end 66.24 77.51) (width 0.5) (layer "F.Cu") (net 1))
 (segment (start 65.15 79.1) (end 65.51 79.1) (width 0.5) (layer "F.Cu") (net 1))
 (segment (start 64.125 79.1) (end 65.15 79.1) (width 0.4) (layer "F.Cu") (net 1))
 (segment (start 66.24 78.37) (end 66.24 77.51) (width 0.5) (layer "F.Cu") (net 1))
 (segment (start 73.115 82.325) (end 73.115 81.825) (width 0.3) (layer "F.Cu") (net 2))
 (segment (start 64.125 81.7) (end 65.15 81.7) (width 0.4) (layer "F.Cu") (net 2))
 (segment (start 73.115 81.45) (end 73.24 81.325) (width 0.3) (layer "F.Cu") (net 2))
 (segment (start 72.455 82.325) (end 72.32 82.46) (width 0.4) (layer "F.Cu") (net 2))
 (segment (start 65.15 81.7) (end 65.8 81.7) (width 0.5) (layer "F.Cu") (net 2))
 (segment (start 74.075 81.825) (end 73.115 81.825) (width 0.3) (layer "F.Cu") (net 2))
 (segment (start 67.2 81.475) (end 66.695 81.475) (width 0.4) (layer "F.Cu") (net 2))
 (segment (start 65.8 81.7) (end 65.8 82.5) (width 0.8) (layer "F.Cu") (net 2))
 (segment (start 68.72 77.64) (end 67.86 77.64) (width 0.5) (layer "F.Cu") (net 2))
 (segment (start 72.13 71.895) (end 72.43 71.595) (width 0.25) (layer "F.Cu") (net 2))
 (segment (start 70.77 82.46) (end 70.77 83.51) (width 0.5) (layer "F.Cu") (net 2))
 (segment (start 66.47 81.7) (end 65.8 81.7) (width 0.4) (layer "F.Cu") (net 2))
 (segment (start 72.635 82.325) (end 72.455 82.325) (width 0.4) (layer "F.Cu") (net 2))
 (segment (start 72.635 82.325) (end 73.115 82.325) (width 0.3) (layer "F.Cu") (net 2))
 (segment (start 71.81 82.46) (end 70.77 82.46) (width 0.5) (layer "F.Cu") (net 2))
 (segment (start 73.115 81.825) (end 73.115 81.45) (width 0.3) (layer "F.Cu") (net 2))
 (segment (start 71.6 72.65) (end 72.13 72.12) (width 0.25) (layer "F.Cu") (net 2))
 (segment (start 67.2 78.675) (end 67.2 77.51) (width 0.4) (layer "F.Cu") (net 2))
 (segment (start 67.73 77.51) (end 67.2 77.51) (width 0.5) (layer "F.Cu") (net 2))
 (segment (start 69.51 77.64) (end 69.51 76.62) (width 0.5) (layer "F.Cu") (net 2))
 (segment (start 68.72 77.64) (end 69.51 77.64) (width 0.5) (layer "F.Cu") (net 2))
 (segment (start 69.51 78.67) (end 69.51 77.64) (width 0.5) (layer "F.Cu") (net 2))
 (segment (start 69.94 73.07) (end 71.18 73.07) (width 0.25) (layer "F.Cu") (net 2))
 (segment (start 67.86 77.64) (end 67.73 77.51) (width 0.5) (layer "F.Cu") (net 2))
 (segment (start 72.32 82.46) (end 71.81 82.46) (width 0.4) (layer "F.Cu") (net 2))
 (segment (start 73.24 81.325) (end 74.075 81.325) (width 0.3) (layer "F.Cu") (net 2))
 (segment (start 71.18 73.07) (end 71.6 72.65) (width 0.25) (layer "F.Cu") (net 2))
 (segment (start 66.695 81.475) (end 66.47 81.7) (width 0.4) (layer "F.Cu") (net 2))
 (segment (start 73.115 82.325) (end 74.075 82.325) (width 0.3) (layer "F.Cu") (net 2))
 (segment (start 72.13 72.12) (end 72.13 71.895) (width 0.25) (layer "F.Cu") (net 2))
 (segment (start 72.43 71.595) (end 72.43 71.1) (width 0.25) (layer "F.Cu") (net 2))
 (via (at 68.72 77.64) (size 0.8) (drill 0.4) (layers "F.Cu" "B.Cu") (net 2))
 (via (at 65.8 81.7) (size 0.8) (drill 0.4) (layers "F.Cu" "B.Cu") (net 2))
 (via (at 65.8 82.5) (size 0.8) (drill 0.4) (layers "F.Cu" "B.Cu") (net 2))
 (segment (start 72.54 83.51) (end 72.81 83.24) (width 0.4) (layer "F.Cu") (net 10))
 (segment (start 72.81 83.24) (end 73.225 82.825) (width 0.3) (layer "F.Cu") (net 10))
 (segment (start 69.66 84.355) (end 69.39 84.085) (width 0.5) (layer "F.Cu") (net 10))
 (segment (start 69.39 84.085) (end 69.39 83.2375) (width 0.5) (layer "F.Cu") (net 10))
 (segment (start 71.42 84.355) (end 69.66 84.355) (width 0.5) (layer "F.Cu") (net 10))
 (segment (start 71.73 83.51) (end 71.73 84.045) (width 0.5) (layer "F.Cu") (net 10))
 (segment (start 71.73 84.045) (end 71.42 84.355) (width 0.5) (layer "F.Cu") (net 10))
 (segment (start 71.73 83.51) (end 72.54 83.51) (width 0.4) (layer "F.Cu") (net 10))
 (segment (start 74.075 82.825) (end 73.225 82.825) (width 0.3) (layer "F.Cu") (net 10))
 (segment (start 80.4875 73.8275) (end 81.105 73.21) (width 0.3) (layer "F.Cu") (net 31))
 (segment (start 80.4875 75.9125) (end 80.4875 73.8275) (width 0.3) (layer "F.Cu") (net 31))
 (segment (start 81.105 73.21) (end 81.565 73.21) (width 0.3) (layer "F.Cu") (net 31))
 (segment (start 80.9875 75.9125) (end 80.9875 74.3975) (width 0.3) (layer "F.Cu") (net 30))
 (segment (start 80.9875 74.3975) (end 81.18 74.205) (width 0.3) (layer "F.Cu") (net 30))
 (segment (start 81.18 74.205) (end 81.565 74.205) (width 0.3) (layer "F.Cu") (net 30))
 (segment (start 79.405 74.72) (end 79.405 74.205) (width 0.3) (layer "F.Cu") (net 32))
 (segment (start 79.4875 74.8025) (end 79.405 74.72) (width 0.3) (layer "F.Cu") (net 32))
 (segment (start 79.4875 75.9125) (end 79.4875 74.8025) (width 0.3) (layer "F.Cu") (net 32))
 (segment (start 73.39 72.24) (end 73.8 72.65) (width 0.25) (layer "F.Cu") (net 3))
 (segment (start 73.035 77.325) (end 74.075 77.325) (width 0.25) (layer "F.Cu") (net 3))
 (segment (start 73.39 71.1) (end 73.39 72.24) (width 0.25) (layer "F.Cu") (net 3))
 (segment (start 73.38 73.07) (end 72.97 73.07) (width 0.25) (layer "F.Cu") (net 3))
 (segment (start 72.7 73.34) (end 72.7 76.99) (width 0.25) (layer "F.Cu") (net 3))
 (segment (start 73.8 72.65) (end 73.38 73.07) (width 0.25) (layer "F.Cu") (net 3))
 (segment (start 72.7 76.99) (end 73.035 77.325) (width 0.25) (layer "F.Cu") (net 3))
 (segment (start 72.97 73.07) (end 72.7 73.34) (width 0.25) (layer "F.Cu") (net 3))
 (segment (start 71.95 75.89) (end 71.95 74.7) (width 0.25) (layer "F.Cu") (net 36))
 (segment (start 69.94 74.03) (end 71.28 74.03) (width 0.25) (layer "F.Cu") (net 36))
 (segment (start 71.28 74.03) (end 71.6 74.35) (width 0.25) (layer "F.Cu") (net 36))
 (segment (start 71.95 74.7) (end 71.6 74.35) (width 0.25) (layer "F.Cu") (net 36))
 (segment (start 69.39 81.6625) (end 70.0475 81.6625) (width 0.5) (layer "F.Cu") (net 9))
 (segment (start 70.21 81.5) (end 70.77 81.5) (width 0.5) (layer "F.Cu") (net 9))
 (segment (start 71.81 81.5) (end 70.77 81.5) (width 0.5) (layer "F.Cu") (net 9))
 (segment (start 72.285 81.5) (end 71.81 81.5) (width 0.4) (layer "F.Cu") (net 9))
 (segment (start 72.585 81.2) (end 72.96 80.825) (width 0.3) (layer "F.Cu") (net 9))
 (segment (start 70.0475 81.6625) (end 70.21 81.5) (width 0.5) (layer "F.Cu") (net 9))
 (segment (start 72.585 81.2) (end 72.285 81.5) (width 0.4) (layer "F.Cu") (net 9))
 (segment (start 72.96 80.825) (end 74.075 80.825) (width 0.3) (layer "F.Cu") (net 9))
 (segment (start 68.51 74.9175) (end 69.4675 74.9175) (width 0.5) (layer "F.Cu") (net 5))
 (segment (start 70.47 75.92) (end 70.47 76.62) (width 0.5) (layer "F.Cu") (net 5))
 (segment (start 70.47 76.62) (end 70.47 77.64) (width 0.5) (layer "F.Cu") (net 5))
 (segment (start 71.22 77.64) (end 71.5 77.92) (width 0.4) (layer "F.Cu") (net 5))
 (segment (start 70.47 77.64) (end 71.22 77.64) (width 0.4) (layer "F.Cu") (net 5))
 (segment (start 71.5 77.92) (end 71.905 78.325) (width 0.3) (layer "F.Cu") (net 5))
 (segment (start 69.4675 74.9175) (end 70.47 75.92) (width 0.5) (layer "F.Cu") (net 5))
 (segment (start 74.075 78.325) (end 71.905 78.325) (width 0.3) (layer "F.Cu") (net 5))
 (segment (start 72.665 80.325) (end 72.35 80.35) (width 0.3) (layer "F.Cu") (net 8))
 (segment (start 64.125 80.4) (end 66.31 80.4) (width 0.4) (layer "F.Cu") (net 8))
 (segment (start 74.075 80.325) (end 72.665 80.325) (width 0.3) (layer "F.Cu") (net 8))
 (segment (start 71.47 78.87) (end 72.705 78.87) (width 0.25) (layer "F.Cu") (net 6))
 (segment (start 73.16 79.325) (end 74.075 79.325) (width 0.25) (layer "F.Cu") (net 6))
 (segment (start 70.53 78.67) (end 71.27 78.67) (width 0.25) (layer "F.Cu") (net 6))
 (segment (start 72.705 78.87) (end 73.16 79.325) (width 0.25) (layer "F.Cu") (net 6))
 (segment (start 71.27 78.67) (end 71.47 78.87) (width 0.25) (layer "F.Cu") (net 6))
 (segment (start 71.95 77.38) (end 71.95 76.91) (width 0.25) (layer "F.Cu") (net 4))
 (segment (start 72.395 77.825) (end 71.95 77.38) (width 0.25) (layer "F.Cu") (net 4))
 (segment (start 74.075 77.825) (end 72.395 77.825) (width 0.25) (layer "F.Cu") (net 4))
 (segment (start 74.075 79.825) (end 72.665 79.825) (width 0.3) (layer "F.Cu") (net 7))
 (segment (start 64.125 79.75) (end 66.31 79.75) (width 0.4) (layer "F.Cu") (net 7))
 (segment (start 72.665 79.825) (end 72.35 79.8) (width 0.3) (layer "F.Cu") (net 7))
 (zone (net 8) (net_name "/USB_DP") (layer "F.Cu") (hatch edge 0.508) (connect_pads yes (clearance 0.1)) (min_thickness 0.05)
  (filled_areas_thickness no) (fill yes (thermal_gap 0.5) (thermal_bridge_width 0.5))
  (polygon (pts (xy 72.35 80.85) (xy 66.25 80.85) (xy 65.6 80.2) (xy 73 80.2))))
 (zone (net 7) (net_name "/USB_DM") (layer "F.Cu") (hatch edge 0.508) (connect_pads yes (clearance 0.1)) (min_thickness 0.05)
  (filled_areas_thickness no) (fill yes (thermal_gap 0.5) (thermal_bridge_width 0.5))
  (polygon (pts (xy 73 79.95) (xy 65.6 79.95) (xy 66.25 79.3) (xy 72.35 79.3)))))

